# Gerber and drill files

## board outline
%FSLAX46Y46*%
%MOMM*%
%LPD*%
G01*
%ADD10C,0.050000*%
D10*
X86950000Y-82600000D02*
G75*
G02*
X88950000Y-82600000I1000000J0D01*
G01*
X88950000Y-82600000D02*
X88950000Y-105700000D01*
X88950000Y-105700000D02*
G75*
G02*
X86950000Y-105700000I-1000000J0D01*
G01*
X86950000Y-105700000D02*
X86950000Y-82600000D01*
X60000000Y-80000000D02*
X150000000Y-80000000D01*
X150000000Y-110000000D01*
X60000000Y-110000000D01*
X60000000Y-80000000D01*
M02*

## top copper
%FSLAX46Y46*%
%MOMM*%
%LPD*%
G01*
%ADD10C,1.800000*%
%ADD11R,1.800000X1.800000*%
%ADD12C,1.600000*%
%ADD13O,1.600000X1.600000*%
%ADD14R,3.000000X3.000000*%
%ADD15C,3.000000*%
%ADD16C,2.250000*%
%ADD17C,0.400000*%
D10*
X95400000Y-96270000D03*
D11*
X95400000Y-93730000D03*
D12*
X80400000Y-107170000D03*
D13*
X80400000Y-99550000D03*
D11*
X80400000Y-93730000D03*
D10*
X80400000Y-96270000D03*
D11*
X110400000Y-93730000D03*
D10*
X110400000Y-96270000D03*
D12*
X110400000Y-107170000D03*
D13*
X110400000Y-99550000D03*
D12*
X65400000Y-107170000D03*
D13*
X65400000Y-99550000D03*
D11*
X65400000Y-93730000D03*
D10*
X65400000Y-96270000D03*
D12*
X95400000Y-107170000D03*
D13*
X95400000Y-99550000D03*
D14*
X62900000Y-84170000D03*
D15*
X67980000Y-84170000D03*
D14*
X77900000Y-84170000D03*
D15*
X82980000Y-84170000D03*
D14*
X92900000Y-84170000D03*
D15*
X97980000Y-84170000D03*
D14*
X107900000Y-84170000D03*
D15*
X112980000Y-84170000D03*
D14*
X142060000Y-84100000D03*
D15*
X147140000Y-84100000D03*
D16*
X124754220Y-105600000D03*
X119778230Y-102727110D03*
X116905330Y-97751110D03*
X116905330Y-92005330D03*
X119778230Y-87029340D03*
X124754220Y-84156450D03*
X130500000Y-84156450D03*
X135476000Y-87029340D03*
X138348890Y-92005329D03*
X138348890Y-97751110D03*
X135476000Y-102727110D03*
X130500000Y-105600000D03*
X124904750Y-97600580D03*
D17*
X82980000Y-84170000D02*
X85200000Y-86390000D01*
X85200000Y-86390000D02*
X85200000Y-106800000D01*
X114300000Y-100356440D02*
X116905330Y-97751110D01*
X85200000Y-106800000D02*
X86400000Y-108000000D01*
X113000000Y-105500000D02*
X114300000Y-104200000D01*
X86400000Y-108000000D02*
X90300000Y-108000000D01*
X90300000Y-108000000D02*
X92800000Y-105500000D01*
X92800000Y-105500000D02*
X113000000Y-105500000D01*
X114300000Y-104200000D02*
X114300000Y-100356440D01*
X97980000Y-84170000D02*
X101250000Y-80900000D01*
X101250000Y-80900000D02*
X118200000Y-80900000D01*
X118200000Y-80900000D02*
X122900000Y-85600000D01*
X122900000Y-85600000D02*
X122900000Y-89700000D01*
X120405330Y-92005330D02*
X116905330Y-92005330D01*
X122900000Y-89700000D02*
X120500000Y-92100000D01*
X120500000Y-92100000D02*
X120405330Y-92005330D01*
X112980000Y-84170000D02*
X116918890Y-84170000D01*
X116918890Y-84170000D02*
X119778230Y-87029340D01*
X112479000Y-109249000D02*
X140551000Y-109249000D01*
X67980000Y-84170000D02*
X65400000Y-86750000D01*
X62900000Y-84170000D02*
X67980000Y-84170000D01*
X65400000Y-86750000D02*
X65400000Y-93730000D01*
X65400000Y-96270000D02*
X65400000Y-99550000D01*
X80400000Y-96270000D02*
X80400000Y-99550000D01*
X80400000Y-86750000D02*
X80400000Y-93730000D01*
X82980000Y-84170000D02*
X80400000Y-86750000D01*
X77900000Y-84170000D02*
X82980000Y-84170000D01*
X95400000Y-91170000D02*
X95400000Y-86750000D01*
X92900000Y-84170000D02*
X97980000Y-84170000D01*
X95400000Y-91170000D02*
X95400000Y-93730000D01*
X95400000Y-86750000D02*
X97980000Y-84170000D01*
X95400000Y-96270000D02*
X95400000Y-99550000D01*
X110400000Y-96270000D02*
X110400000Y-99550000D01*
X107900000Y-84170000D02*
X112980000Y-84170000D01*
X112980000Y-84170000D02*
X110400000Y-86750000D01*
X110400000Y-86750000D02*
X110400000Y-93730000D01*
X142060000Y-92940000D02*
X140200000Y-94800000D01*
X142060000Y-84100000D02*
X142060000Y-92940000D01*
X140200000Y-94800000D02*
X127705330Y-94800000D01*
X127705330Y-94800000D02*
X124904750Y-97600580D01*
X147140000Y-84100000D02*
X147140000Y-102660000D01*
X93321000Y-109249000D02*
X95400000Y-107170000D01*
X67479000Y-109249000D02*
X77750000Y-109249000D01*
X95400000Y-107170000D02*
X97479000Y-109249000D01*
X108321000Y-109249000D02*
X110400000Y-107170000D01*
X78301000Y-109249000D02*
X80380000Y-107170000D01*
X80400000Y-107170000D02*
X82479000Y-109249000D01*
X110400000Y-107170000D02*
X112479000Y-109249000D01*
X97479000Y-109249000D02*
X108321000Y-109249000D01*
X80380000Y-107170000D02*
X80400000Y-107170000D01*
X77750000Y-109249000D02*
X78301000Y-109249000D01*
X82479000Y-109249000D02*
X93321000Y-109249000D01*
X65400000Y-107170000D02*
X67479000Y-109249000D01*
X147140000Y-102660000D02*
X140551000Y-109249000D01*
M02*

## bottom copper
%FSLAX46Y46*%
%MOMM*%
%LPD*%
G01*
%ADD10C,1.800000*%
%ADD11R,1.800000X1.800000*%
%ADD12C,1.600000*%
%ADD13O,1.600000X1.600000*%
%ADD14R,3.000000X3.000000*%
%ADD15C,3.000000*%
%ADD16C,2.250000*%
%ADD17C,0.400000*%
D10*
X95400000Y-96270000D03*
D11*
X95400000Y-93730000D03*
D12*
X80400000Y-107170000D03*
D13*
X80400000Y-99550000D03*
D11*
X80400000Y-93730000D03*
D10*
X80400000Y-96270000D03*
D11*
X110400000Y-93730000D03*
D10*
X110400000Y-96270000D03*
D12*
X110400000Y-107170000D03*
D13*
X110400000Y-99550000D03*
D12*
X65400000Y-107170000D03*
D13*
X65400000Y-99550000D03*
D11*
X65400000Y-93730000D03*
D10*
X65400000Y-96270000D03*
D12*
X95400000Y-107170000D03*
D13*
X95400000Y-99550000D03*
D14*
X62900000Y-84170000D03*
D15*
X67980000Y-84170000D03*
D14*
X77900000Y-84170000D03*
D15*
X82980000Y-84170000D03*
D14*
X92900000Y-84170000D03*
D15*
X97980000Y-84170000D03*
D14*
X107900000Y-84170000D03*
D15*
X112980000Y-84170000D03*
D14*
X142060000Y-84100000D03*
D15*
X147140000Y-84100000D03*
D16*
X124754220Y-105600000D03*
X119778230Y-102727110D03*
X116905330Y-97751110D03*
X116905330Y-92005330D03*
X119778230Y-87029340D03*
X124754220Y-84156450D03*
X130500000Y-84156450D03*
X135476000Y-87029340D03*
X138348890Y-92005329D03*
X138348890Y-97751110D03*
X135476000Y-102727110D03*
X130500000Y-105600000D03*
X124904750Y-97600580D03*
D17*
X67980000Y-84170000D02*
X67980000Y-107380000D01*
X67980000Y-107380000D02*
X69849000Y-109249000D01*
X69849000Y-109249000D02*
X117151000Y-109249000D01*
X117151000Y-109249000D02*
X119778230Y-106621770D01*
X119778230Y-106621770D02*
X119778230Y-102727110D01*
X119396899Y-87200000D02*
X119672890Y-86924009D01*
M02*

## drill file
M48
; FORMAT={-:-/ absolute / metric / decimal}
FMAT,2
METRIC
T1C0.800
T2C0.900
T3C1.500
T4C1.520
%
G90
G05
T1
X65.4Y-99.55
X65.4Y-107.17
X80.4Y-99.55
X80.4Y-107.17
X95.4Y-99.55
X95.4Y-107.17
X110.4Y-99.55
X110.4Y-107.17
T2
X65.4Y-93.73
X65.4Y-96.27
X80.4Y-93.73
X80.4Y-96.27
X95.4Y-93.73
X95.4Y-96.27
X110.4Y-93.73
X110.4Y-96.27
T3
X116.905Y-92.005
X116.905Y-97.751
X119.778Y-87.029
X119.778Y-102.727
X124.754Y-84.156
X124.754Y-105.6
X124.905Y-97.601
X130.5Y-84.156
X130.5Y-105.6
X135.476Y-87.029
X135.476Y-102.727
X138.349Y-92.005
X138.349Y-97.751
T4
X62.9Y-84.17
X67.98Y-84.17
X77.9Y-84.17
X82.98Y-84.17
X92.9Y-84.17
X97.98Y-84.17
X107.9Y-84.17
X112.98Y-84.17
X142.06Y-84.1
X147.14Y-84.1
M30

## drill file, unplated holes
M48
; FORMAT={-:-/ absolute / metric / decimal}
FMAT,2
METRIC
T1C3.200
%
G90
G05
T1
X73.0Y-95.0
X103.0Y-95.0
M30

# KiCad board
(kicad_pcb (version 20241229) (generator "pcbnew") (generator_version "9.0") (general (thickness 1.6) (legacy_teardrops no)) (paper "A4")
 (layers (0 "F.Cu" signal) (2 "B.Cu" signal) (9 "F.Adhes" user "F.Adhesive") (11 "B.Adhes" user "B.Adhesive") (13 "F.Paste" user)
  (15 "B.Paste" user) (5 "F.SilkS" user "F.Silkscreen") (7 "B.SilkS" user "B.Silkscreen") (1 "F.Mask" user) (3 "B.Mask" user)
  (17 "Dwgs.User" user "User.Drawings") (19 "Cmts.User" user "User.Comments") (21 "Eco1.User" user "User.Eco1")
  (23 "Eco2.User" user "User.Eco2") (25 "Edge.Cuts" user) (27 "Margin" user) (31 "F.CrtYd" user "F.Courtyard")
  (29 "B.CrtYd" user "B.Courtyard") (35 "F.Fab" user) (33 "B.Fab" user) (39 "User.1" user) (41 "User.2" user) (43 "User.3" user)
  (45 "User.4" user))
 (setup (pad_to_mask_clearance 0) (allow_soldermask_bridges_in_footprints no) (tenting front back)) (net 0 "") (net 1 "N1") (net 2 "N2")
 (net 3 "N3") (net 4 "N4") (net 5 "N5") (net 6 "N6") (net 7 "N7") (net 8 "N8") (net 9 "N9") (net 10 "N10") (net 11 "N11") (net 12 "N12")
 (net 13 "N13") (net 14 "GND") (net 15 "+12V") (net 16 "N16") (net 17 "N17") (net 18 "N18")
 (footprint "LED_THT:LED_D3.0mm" (layer "F.Cu") (at 95.4 93.73 -90)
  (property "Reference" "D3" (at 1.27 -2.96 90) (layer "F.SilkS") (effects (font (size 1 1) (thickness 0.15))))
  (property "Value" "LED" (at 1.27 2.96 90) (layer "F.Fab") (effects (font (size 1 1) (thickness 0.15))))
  (pad "1" thru_hole rect (at 0 0 270) (size 1.8 1.8) (drill 0.9) (layers "*.Cu" "*.Mask") (remove_unused_layers no) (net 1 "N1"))
  (pad "2" thru_hole circle (at 2.54 0 270) (size 1.8 1.8) (drill 0.9) (layers "*.Cu" "*.Mask") (remove_unused_layers no) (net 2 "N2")))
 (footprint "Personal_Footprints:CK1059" (layer "F.Cu") (at 124.75422 105.6)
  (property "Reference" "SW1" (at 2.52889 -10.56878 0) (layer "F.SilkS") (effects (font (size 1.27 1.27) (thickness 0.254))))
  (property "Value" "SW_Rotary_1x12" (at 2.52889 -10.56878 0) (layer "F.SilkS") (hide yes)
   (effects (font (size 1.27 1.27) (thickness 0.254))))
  (pad "1" thru_hole circle (at 0 0) (size 2.25 2.25) (drill 1.5) (layers "*.Cu" "*.Mask") (remove_unused_layers no) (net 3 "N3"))
  (pad "2" thru_hole circle (at -4.97599 -2.87289) (size 2.25 2.25) (drill 1.5) (layers "*.Cu" "*.Mask") (remove_unused_layers no)
   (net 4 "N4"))
  (pad "3" thru_hole circle (at -7.84889 -7.84889) (size 2.25 2.25) (drill 1.5) (layers "*.Cu" "*.Mask") (remove_unused_layers no)
   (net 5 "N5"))
  (pad "4" thru_hole circle (at -7.84889 -13.59467) (size 2.25 2.25) (drill 1.5) (layers "*.Cu" "*.Mask") (remove_unused_layers no)
   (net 1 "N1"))
  (pad "5" thru_hole circle (at -4.97599 -18.57066) (size 2.25 2.25) (drill 1.5) (layers "*.Cu" "*.Mask") (remove_unused_layers no)
   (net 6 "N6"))
  (pad "6" thru_hole circle (at 0 -21.44355) (size 2.25 2.25) (drill 1.5) (layers "*.Cu" "*.Mask") (remove_unused_layers no) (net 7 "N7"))
  (pad "7" thru_hole circle (at 5.74578 -21.44355) (size 2.25 2.25) (drill 1.5) (layers "*.Cu" "*.Mask") (remove_unused_layers no)
   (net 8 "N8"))
  (pad "8" thru_hole circle (at 10.72178 -18.57066) (size 2.25 2.25) (drill 1.5) (layers "*.Cu" "*.Mask") (remove_unused_layers no)
   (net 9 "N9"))
  (pad "9" thru_hole circle (at 13.59467 -13.594671) (size 2.25 2.25) (drill 1.5) (layers "*.Cu" "*.Mask") (remove_unused_layers no)
   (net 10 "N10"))
  (pad "10" thru_hole circle (at 13.59467 -7.84889) (size 2.25 2.25) (drill 1.5) (layers "*.Cu" "*.Mask") (remove_unused_layers no)
   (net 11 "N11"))
  (pad "11" thru_hole circle (at 10.72178 -2.87289) (size 2.25 2.25) (drill 1.5) (layers "*.Cu" "*.Mask") (remove_unused_layers no)
   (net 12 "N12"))
  (pad "12" thru_hole circle (at 5.74578 0) (size 2.25 2.25) (drill 1.5) (layers "*.Cu" "*.Mask") (remove_unused_layers no) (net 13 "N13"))
  (pad "13" thru_hole circle (at 0.15053 -7.99942) (size 2.25 2.25) (drill 1.5) (layers "*.Cu" "*.Mask") (remove_unused_layers no)
   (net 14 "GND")))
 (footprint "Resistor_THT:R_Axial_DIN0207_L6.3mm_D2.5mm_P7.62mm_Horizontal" (layer "F.Cu") (at 80.4 107.17 90)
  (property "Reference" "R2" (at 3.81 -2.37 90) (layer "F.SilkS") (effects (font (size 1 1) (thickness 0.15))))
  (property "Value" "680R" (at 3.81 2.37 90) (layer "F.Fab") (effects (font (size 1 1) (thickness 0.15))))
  (pad "1" thru_hole circle (at 0 0 90) (size 1.6 1.6) (drill 0.8) (layers "*.Cu" "*.Mask") (remove_unused_layers no) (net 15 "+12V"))
  (pad "2" thru_hole oval (at 7.62 0 90) (size 1.6 1.6) (drill 0.8) (layers "*.Cu" "*.Mask") (remove_unused_layers no) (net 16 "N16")))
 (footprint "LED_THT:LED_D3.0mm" (layer "F.Cu") (at 80.4 93.73 -90)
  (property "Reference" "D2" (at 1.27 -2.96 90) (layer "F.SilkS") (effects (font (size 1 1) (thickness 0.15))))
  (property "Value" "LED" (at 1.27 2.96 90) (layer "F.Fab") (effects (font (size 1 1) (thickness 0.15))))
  (pad "1" thru_hole rect (at 0 0 270) (size 1.8 1.8) (drill 0.9) (layers "*.Cu" "*.Mask") (remove_unused_layers no) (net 5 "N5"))
  (pad "2" thru_hole circle (at 2.54 0 270) (size 1.8 1.8) (drill 0.9) (layers "*.Cu" "*.Mask") (remove_unused_layers no) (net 16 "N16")))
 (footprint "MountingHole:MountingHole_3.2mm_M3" (layer "F.Cu") (at 103 95)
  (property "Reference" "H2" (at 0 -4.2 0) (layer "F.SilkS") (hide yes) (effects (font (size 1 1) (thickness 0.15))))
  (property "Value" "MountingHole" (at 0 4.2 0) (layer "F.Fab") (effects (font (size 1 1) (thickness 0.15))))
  (pad "" np_thru_hole circle (at 0 0) (size 3.2 3.2) (drill 3.2) (layers "*.Cu" "*.Mask")))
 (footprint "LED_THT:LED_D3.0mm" (layer "F.Cu") (at 110.4 93.73 -90)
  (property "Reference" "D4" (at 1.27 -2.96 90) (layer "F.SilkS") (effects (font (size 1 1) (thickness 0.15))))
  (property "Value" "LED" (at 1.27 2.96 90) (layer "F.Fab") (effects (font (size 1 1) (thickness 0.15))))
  (pad "1" thru_hole rect (at 0 0 270) (size 1.8 1.8) (drill 0.9) (layers "*.Cu" "*.Mask") (remove_unused_layers no) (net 6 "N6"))
  (pad "2" thru_hole circle (at 2.54 0 270) (size 1.8 1.8) (drill 0.9) (layers "*.Cu" "*.Mask") (remove_unused_layers no) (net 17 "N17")))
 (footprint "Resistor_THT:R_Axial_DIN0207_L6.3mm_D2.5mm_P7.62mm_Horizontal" (layer "F.Cu") (at 110.4 107.17 90)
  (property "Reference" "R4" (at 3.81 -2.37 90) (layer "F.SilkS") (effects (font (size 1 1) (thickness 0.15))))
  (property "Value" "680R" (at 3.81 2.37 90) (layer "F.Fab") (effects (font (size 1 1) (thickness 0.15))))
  (pad "1" thru_hole circle (at 0 0 90) (size 1.6 1.6) (drill 0.8) (layers "*.Cu" "*.Mask") (remove_unused_layers no) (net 15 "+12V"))
  (pad "2" thru_hole oval (at 7.62 0 90) (size 1.6 1.6) (drill 0.8) (layers "*.Cu" "*.Mask") (remove_unused_layers no) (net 17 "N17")))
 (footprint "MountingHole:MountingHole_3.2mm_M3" (layer "F.Cu") (at 73 95)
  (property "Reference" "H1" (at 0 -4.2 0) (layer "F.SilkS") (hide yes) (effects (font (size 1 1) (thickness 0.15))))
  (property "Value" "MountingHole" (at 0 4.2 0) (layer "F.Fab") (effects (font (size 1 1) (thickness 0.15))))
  (pad "" np_thru_hole circle (at 0 0) (size 3.2 3.2) (drill 3.2) (layers "*.Cu" "*.Mask")))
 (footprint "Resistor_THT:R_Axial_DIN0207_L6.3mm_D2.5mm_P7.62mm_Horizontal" (layer "F.Cu") (at 65.4 107.17 90)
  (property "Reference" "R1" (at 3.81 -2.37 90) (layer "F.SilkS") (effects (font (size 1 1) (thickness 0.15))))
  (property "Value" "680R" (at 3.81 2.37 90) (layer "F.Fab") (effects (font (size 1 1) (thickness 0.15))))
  (pad "1" thru_hole circle (at 0 0 90) (size 1.6 1.6) (drill 0.8) (layers "*.Cu" "*.Mask") (remove_unused_layers no) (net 15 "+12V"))
  (pad "2" thru_hole oval (at 7.62 0 90) (size 1.6 1.6) (drill 0.8) (layers "*.Cu" "*.Mask") (remove_unused_layers no) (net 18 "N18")))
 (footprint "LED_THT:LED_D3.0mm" (layer "F.Cu") (at 65.4 93.73 -90)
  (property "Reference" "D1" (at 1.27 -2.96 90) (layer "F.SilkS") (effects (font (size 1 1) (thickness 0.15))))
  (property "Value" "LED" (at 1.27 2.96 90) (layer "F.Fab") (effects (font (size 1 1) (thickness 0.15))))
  (pad "1" thru_hole rect (at 0 0 270) (size 1.8 1.8) (drill 0.9) (layers "*.Cu" "*.Mask") (remove_unused_layers no) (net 4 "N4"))
  (pad "2" thru_hole circle (at 2.54 0 270) (size 1.8 1.8) (drill 0.9) (layers "*.Cu" "*.Mask") (remove_unused_layers no) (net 18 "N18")))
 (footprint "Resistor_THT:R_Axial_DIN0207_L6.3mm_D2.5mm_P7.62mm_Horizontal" (layer "F.Cu") (at 95.4 107.17 90)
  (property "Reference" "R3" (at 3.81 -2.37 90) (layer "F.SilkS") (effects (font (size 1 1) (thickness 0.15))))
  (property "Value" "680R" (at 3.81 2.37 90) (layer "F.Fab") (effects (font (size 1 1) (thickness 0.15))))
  (pad "1" thru_hole circle (at 0 0 90) (size 1.6 1.6) (drill 0.8) (layers "*.Cu" "*.Mask") (remove_unused_layers no) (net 15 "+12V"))
  (pad "2" thru_hole oval (at 7.62 0 90) (size 1.6 1.6) (drill 0.8) (layers "*.Cu" "*.Mask") (remove_unused_layers no) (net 2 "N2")))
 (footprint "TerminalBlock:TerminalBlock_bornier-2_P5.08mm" (layer "B.Cu") (at 62.9 84.17)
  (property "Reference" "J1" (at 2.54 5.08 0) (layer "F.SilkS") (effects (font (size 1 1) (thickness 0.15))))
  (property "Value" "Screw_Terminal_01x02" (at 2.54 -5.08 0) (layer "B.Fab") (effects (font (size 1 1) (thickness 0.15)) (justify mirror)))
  (pad "1" thru_hole rect (at 0 0) (size 3 3) (drill 1.52) (layers "*.Cu" "*.Mask") (remove_unused_layers no) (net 4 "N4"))
  (pad "2" thru_hole circle (at 5.08 0) (size 3 3) (drill 1.52) (layers "*.Cu" "*.Mask") (remove_unused_layers no) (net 4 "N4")))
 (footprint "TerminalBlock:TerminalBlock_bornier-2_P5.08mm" (layer "B.Cu") (at 77.9 84.17)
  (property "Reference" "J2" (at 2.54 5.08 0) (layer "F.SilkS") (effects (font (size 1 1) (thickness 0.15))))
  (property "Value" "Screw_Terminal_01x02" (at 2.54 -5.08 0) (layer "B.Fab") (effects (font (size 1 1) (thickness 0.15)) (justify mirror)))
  (pad "1" thru_hole rect (at 0 0) (size 3 3) (drill 1.52) (layers "*.Cu" "*.Mask") (remove_unused_layers no) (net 5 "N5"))
  (pad "2" thru_hole circle (at 5.08 0) (size 3 3) (drill 1.52) (layers "*.Cu" "*.Mask") (remove_unused_layers no) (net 5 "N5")))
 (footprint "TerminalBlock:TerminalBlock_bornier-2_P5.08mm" (layer "B.Cu") (at 92.9 84.17)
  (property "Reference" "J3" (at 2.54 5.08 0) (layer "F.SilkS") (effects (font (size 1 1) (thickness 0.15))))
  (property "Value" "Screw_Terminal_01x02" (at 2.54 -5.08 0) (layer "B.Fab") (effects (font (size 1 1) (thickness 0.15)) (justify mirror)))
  (pad "1" thru_hole rect (at 0 0) (size 3 3) (drill 1.52) (layers "*.Cu" "*.Mask") (remove_unused_layers no) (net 1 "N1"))
  (pad "2" thru_hole circle (at 5.08 0) (size 3 3) (drill 1.52) (layers "*.Cu" "*.Mask") (remove_unused_layers no) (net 1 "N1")))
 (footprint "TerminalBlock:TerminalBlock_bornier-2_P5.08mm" (layer "B.Cu") (at 107.9 84.17)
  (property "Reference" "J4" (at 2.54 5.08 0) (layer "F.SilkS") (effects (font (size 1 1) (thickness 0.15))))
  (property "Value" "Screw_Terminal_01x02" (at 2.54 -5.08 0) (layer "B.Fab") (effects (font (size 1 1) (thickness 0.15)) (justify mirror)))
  (pad "1" thru_hole rect (at 0 0) (size 3 3) (drill 1.52) (layers "*.Cu" "*.Mask") (remove_unused_layers no) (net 6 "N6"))
  (pad "2" thru_hole circle (at 5.08 0) (size 3 3) (drill 1.52) (layers "*.Cu" "*.Mask") (remove_unused_layers no) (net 6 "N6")))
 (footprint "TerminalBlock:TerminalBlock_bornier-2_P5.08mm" (layer "B.Cu") (at 142.06 84.1)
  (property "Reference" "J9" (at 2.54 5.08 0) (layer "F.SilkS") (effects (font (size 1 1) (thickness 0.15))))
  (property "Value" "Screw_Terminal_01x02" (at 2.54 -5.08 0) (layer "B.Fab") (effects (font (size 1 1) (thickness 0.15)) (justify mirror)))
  (pad "1" thru_hole rect (at 0 0) (size 3 3) (drill 1.52) (layers "*.Cu" "*.Mask") (remove_unused_layers no) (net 14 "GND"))
  (pad "2" thru_hole circle (at 5.08 0) (size 3 3) (drill 1.52) (layers "*.Cu" "*.Mask") (remove_unused_layers no) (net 15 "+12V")))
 (gr_arc (start 86.95 82.6) (mid 87.95 81.6) (end 88.95 82.6) (stroke (width 0.05) (type default)) (layer "Edge.Cuts"))
 (gr_line (start 88.95 82.6) (end 88.95 105.7) (stroke (width 0.05) (type default)) (layer "Edge.Cuts"))
 (gr_arc (start 88.95 105.7) (mid 87.95 106.7) (end 86.95 105.7) (stroke (width 0.05) (type default)) (layer "Edge.Cuts"))
 (gr_line (start 86.95 105.7) (end 86.95 82.6) (stroke (width 0.05) (type default)) (layer "Edge.Cuts"))
 (gr_rect (start 60 80) (end 150 110) (stroke (width 0.05) (type solid)) (fill no) (layer "Edge.Cuts"))
 (segment (start 67.98 84.17) (end 65.4 86.75) (width 0.4) (layer "F.Cu") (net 4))
 (segment (start 62.9 84.17) (end 67.98 84.17) (width 0.4) (layer "F.Cu") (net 4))
 (segment (start 65.4 86.75) (end 65.4 93.73) (width 0.4) (layer "F.Cu") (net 4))
 (segment (start 117.151 109.249) (end 119.77823 106.62177) (width 0.4) (layer "B.Cu") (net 4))
 (segment (start 67.98 107.38) (end 69.849 109.249) (width 0.4) (layer "B.Cu") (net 4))
 (segment (start 119.77823 106.62177) (end 119.77823 102.72711) (width 0.4) (layer "B.Cu") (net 4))
 (segment (start 67.98 84.17) (end 67.98 107.38) (width 0.4) (layer "B.Cu") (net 4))
 (segment (start 69.849 109.249) (end 117.151 109.249) (width 0.4) (layer "B.Cu") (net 4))
 (segment (start 65.4 96.27) (end 65.4 99.55) (width 0.4) (layer "F.Cu") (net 18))
 (segment (start 80.4 96.27) (end 80.4 99.55) (width 0.4) (layer "F.Cu") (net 16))
 (segment (start 82.98 84.17) (end 85.2 86.39) (width 0.4) (layer "F.Cu") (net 5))
 (segment (start 113 105.5) (end 114.3 104.2) (width 0.4) (layer "F.Cu") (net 5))
 (segment (start 85.2 86.39) (end 85.2 106.8) (width 0.4) (layer "F.Cu") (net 5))
 (segment (start 90.3 108) (end 92.8 105.5) (width 0.4) (layer "F.Cu") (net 5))
 (segment (start 114.3 104.2) (end 114.3 100.35644) (width 0.4) (layer "F.Cu") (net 5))
 (segment (start 85.2 106.8) (end 86.4 108) (width 0.4) (layer "F.Cu") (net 5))
 (segment (start 80.4 86.75) (end 80.4 93.73) (width 0.4) (layer "F.Cu") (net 5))
 (segment (start 114.3 100.35644) (end 116.90533 97.75111) (width 0.4) (layer "F.Cu") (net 5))
 (segment (start 82.98 84.17) (end 80.4 86.75) (width 0.4) (layer "F.Cu") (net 5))
 (segment (start 92.8 105.5) (end 113 105.5) (width 0.4) (layer "F.Cu") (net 5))
 (segment (start 77.9 84.17) (end 82.98 84.17) (width 0.4) (layer "F.Cu") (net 5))
 (segment (start 86.4 108) (end 90.3 108) (width 0.4) (layer "F.Cu") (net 5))
 (segment (start 95.4 91.17) (end 95.4 86.75) (width 0.4) (layer "F.Cu") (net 1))
 (segment (start 92.9 84.17) (end 97.98 84.17) (width 0.4) (layer "F.Cu") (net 1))
 (segment (start 95.4 91.17) (end 95.4 93.73) (width 0.4) (layer "F.Cu") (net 1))
 (segment (start 120.40533 92.00533) (end 116.90533 92.00533) (width 0.4) (layer "F.Cu") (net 1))
 (segment (start 120.5 92.1) (end 120.40533 92.00533) (width 0.4) (layer "F.Cu") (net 1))
 (segment (start 118.2 80.9) (end 122.9 85.6) (width 0.4) (layer "F.Cu") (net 1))
 (segment (start 97.98 84.17) (end 101.25 80.9) (width 0.4) (layer "F.Cu") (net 1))
 (segment (start 122.9 89.7) (end 120.5 92.1) (width 0.4) (layer "F.Cu") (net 1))
 (segment (start 122.9 85.6) (end 122.9 89.7) (width 0.4) (layer "F.Cu") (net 1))
 (segment (start 101.25 80.9) (end 118.2 80.9) (width 0.4) (layer "F.Cu") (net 1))
 (segment (start 95.4 86.75) (end 97.98 84.17) (width 0.4) (layer "F.Cu") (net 1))
 (segment (start 95.4 96.27) (end 95.4 99.55) (width 0.4) (layer "F.Cu") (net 2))
 (segment (start 110.4 96.27) (end 110.4 99.55) (width 0.4) (layer "F.Cu") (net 17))
 (segment (start 112.98 84.17) (end 116.91889 84.17) (width 0.4) (layer "F.Cu") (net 6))
 (segment (start 107.9 84.17) (end 112.98 84.17) (width 0.4) (layer "F.Cu") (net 6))
 (segment (start 112.98 84.17) (end 110.4 86.75) (width 0.4) (layer "F.Cu") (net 6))
 (segment (start 116.91889 84.17) (end 119.77823 87.02934) (width 0.4) (layer "F.Cu") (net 6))
 (segment (start 110.4 86.75) (end 110.4 93.73) (width 0.4) (layer "F.Cu") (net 6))
 (segment (start 119.396899 87.2) (end 119.67289 86.924009) (width 0.4) (layer "B.Cu") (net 6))
 (segment (start 142.06 92.94) (end 140.2 94.8) (width 0.4) (layer "F.Cu") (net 14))
 (segment (start 142.06 84.1) (end 142.06 92.94) (width 0.4) (layer "F.Cu") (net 14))
 (segment (start 140.2 94.8) (end 127.70533 94.8) (width 0.4) (layer "F.Cu") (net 14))
 (segment (start 127.70533 94.8) (end 124.90475 97.60058) (width 0.4) (layer "F.Cu") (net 14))
 (segment (start 147.14 84.1) (end 147.14 102.66) (width 0.4) (layer "F.Cu") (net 15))
 (segment (start 112.479 109.249) (end 140.551 109.249) (width 0.4) (layer "F.Cu") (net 15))
 (segment (start 93.321 109.249) (end 95.4 107.17) (width 0.4) (layer "F.Cu") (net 15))
 (segment (start 67.479 109.249) (end 77.75 109.249) (width 0.4) (layer "F.Cu") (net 15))
 (segment (start 95.4 107.17) (end 97.479 109.249) (width 0.4) (layer "F.Cu") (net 15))
 (segment (start 108.321 109.249) (end 110.4 107.17) (width 0.4) (layer "F.Cu") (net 15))
 (segment (start 78.301 109.249) (end 80.38 107.17) (width 0.4) (layer "F.Cu") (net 15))
 (segment (start 80.4 107.17) (end 82.479 109.249) (width 0.4) (layer "F.Cu") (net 15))
 (segment (start 110.4 107.17) (end 112.479 109.249) (width 0.4) (layer "F.Cu") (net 15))
 (segment (start 97.479 109.249) (end 108.321 109.249) (width 0.4) (layer "F.Cu") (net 15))
 (segment (start 80.38 107.17) (end 80.4 107.17) (width 0.4) (layer "F.Cu") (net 15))
 (segment (start 77.75 109.249) (end 78.301 109.249) (width 0.4) (layer "F.Cu") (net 15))
 (segment (start 82.479 109.249) (end 93.321 109.249) (width 0.4) (layer "F.Cu") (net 15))
 (segment (start 65.4 107.17) (end 67.479 109.249) (width 0.4) (layer "F.Cu") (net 15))
 (segment (start 147.14 102.66) (end 140.551 109.249) (width 0.4) (layer "F.Cu") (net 15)))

